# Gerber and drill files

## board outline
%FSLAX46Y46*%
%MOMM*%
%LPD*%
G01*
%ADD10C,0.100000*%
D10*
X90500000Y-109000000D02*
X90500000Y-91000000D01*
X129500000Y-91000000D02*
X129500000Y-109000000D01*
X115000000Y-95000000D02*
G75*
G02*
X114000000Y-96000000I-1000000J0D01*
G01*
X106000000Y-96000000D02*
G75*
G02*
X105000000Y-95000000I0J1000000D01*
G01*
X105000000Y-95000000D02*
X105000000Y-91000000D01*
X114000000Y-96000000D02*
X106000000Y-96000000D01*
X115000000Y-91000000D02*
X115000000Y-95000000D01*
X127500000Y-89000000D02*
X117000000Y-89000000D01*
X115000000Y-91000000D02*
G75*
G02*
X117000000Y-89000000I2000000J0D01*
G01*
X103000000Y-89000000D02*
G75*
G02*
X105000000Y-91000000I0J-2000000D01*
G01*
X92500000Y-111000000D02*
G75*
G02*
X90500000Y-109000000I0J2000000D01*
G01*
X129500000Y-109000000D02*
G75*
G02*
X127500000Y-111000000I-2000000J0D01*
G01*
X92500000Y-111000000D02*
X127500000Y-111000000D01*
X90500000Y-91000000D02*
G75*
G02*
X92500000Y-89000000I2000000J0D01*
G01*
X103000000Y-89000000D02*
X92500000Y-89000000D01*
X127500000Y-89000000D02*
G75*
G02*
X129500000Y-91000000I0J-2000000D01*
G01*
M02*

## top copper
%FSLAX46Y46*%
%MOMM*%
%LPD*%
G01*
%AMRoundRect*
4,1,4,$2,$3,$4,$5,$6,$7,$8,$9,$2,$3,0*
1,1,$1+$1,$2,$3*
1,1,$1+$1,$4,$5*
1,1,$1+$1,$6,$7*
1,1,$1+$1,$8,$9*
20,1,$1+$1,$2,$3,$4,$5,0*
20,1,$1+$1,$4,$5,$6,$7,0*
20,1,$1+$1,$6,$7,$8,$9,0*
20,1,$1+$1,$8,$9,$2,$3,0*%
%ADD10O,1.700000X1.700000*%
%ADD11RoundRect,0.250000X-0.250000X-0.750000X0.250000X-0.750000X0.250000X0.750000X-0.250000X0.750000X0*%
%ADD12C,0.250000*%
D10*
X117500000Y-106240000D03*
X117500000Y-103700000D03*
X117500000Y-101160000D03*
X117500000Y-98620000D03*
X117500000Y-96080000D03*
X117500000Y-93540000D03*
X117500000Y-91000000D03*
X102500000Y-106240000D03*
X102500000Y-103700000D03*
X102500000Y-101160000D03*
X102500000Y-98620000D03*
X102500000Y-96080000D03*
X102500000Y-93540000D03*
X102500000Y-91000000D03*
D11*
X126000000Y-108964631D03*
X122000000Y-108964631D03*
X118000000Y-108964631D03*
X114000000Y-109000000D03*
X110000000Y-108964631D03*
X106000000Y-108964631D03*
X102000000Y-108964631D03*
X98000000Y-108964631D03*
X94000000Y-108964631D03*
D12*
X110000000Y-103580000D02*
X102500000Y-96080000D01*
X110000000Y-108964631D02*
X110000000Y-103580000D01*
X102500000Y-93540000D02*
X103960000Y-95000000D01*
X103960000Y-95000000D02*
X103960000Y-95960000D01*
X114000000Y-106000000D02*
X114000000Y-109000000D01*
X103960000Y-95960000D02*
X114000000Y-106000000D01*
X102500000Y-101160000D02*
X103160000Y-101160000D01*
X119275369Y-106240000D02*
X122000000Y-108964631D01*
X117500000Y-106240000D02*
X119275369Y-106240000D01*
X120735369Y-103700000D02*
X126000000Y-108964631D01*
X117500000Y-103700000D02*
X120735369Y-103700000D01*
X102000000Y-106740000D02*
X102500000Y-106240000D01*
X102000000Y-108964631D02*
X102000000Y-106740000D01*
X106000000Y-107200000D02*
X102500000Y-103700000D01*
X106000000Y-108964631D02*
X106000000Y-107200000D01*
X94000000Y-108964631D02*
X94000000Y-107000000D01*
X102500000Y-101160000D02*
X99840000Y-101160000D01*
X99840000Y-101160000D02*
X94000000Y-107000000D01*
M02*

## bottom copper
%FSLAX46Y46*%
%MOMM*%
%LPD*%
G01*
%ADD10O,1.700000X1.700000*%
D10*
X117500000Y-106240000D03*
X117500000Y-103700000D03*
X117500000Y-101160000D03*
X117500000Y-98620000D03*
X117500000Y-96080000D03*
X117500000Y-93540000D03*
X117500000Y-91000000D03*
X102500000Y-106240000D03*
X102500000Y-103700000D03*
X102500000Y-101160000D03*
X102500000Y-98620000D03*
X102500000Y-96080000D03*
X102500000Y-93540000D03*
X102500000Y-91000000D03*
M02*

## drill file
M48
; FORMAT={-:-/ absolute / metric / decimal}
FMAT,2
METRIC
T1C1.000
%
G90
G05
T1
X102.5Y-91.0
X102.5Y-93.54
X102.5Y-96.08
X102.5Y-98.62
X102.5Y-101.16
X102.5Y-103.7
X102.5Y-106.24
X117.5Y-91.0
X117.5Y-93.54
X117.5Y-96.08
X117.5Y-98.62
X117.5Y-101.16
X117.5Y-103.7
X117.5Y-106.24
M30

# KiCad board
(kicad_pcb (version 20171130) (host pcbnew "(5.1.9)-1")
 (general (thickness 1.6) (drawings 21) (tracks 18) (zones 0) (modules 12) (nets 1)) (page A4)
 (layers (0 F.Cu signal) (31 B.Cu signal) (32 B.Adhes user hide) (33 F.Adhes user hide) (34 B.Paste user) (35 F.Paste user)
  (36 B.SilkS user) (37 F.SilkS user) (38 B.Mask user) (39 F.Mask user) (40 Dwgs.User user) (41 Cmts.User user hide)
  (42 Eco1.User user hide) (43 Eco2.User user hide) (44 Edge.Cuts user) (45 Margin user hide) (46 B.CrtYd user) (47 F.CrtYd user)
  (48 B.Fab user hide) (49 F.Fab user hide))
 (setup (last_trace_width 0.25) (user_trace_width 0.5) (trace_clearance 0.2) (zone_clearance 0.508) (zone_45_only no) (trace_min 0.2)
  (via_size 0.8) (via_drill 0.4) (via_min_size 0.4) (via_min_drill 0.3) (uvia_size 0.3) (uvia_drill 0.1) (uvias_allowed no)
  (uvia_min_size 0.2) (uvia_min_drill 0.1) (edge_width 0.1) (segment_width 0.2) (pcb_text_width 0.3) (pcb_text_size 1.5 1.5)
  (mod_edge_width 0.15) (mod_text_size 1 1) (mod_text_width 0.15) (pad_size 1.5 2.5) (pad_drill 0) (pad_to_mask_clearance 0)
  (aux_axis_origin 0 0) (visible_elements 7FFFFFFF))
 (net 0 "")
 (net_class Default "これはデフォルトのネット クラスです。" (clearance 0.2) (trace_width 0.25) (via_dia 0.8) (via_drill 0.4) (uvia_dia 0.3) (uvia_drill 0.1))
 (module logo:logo (layer F.Cu) (at 96.5 99 90)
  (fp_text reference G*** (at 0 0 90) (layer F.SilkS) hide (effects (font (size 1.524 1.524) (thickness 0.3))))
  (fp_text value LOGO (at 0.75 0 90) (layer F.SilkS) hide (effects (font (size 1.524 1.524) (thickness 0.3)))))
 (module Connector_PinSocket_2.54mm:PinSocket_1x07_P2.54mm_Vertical (layer F.Cu) (at 117.5 91)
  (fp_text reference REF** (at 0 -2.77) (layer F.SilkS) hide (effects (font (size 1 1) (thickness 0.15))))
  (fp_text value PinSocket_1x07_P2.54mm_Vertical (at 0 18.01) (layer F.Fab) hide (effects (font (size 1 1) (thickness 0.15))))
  (pad 7 thru_hole oval (at 0 15.24) (size 1.7 1.7) (drill 1) (layers *.Cu *.Mask))
  (pad 6 thru_hole oval (at 0 12.7) (size 1.7 1.7) (drill 1) (layers *.Cu *.Mask))
  (pad 5 thru_hole oval (at 0 10.16) (size 1.7 1.7) (drill 1) (layers *.Cu *.Mask))
  (pad 4 thru_hole oval (at 0 7.62) (size 1.7 1.7) (drill 1) (layers *.Cu *.Mask))
  (pad 3 thru_hole oval (at 0 5.08) (size 1.7 1.7) (drill 1) (layers *.Cu *.Mask))
  (pad 2 thru_hole oval (at 0 2.54) (size 1.7 1.7) (drill 1) (layers *.Cu *.Mask))
  (pad 1 thru_hole oval (at 0 0) (size 1.7 1.7) (drill 1) (layers *.Cu *.Mask)))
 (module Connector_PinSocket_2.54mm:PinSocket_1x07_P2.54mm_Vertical (layer F.Cu) (at 102.5 91)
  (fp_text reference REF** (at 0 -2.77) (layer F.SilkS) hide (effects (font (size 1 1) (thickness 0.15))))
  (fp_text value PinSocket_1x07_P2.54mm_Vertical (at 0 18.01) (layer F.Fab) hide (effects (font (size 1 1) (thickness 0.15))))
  (pad 8 thru_hole oval (at 0 15.24) (size 1.7 1.7) (drill 1) (layers *.Cu *.Mask))
  (pad 9 thru_hole oval (at 0 12.7) (size 1.7 1.7) (drill 1) (layers *.Cu *.Mask))
  (pad 10 thru_hole oval (at 0 10.16) (size 1.7 1.7) (drill 1) (layers *.Cu *.Mask))
  (pad 11 thru_hole oval (at 0 7.62) (size 1.7 1.7) (drill 1) (layers *.Cu *.Mask))
  (pad 12 thru_hole oval (at 0 5.08) (size 1.7 1.7) (drill 1) (layers *.Cu *.Mask))
  (pad 13 thru_hole oval (at 0 2.54) (size 1.7 1.7) (drill 1) (layers *.Cu *.Mask))
  (pad 14 thru_hole oval (at 0 0) (size 1.7 1.7) (drill 1) (layers *.Cu *.Mask)))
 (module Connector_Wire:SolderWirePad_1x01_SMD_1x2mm (layer F.Cu) (at 126 108.964631)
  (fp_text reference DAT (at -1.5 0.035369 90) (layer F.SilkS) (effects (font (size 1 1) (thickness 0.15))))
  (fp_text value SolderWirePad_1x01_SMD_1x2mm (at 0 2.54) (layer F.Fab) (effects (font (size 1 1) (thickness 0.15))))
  (pad 9 smd roundrect (at 0 0) (size 1 2) (layers F.Cu F.Paste F.Mask) (roundrect_rratio 0.25)))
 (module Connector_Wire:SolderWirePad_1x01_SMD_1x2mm (layer F.Cu) (at 122 108.964631)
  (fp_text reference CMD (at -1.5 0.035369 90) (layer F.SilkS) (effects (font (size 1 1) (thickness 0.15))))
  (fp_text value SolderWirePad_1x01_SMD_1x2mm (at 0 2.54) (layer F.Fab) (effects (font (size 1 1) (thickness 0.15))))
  (pad 8 smd roundrect (at 0 0) (size 1 2) (layers F.Cu F.Paste F.Mask) (roundrect_rratio 0.25)))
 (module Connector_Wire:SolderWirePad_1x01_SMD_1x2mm (layer F.Cu) (at 118 108.964631)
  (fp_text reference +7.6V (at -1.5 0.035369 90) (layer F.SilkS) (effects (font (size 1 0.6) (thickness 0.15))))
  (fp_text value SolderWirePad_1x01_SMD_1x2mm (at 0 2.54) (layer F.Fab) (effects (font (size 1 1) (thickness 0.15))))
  (pad 7 smd roundrect (at 0 0) (size 1 2) (layers F.Cu F.Paste F.Mask) (roundrect_rratio 0.25)))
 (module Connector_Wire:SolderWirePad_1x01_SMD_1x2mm (layer F.Cu) (at 114 109)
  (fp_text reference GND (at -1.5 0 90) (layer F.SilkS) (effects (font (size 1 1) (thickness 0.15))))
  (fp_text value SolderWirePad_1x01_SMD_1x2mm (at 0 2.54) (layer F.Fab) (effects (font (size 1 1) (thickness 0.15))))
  (pad 6 smd roundrect (at 0 0) (size 1 2) (layers F.Cu F.Paste F.Mask) (roundrect_rratio 0.25)))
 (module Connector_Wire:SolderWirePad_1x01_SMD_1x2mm (layer F.Cu) (at 110 108.964631)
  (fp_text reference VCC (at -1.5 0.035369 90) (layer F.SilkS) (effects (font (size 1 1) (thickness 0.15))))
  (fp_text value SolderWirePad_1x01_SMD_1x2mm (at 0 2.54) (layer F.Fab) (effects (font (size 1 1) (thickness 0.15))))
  (pad 5 smd roundrect (at 0 0) (size 1 2) (layers F.Cu F.Paste F.Mask) (roundrect_rratio 0.25)))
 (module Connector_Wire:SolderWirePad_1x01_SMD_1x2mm (layer F.Cu) (at 106 108.964631)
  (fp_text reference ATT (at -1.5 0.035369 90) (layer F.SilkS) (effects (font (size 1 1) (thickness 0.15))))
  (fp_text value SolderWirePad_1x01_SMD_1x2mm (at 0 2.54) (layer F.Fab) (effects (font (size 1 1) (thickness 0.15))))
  (pad 4 smd roundrect (at 0 0) (size 1 2) (layers F.Cu F.Paste F.Mask) (roundrect_rratio 0.25)))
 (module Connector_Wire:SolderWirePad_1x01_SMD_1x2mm (layer F.Cu) (at 102 108.964631)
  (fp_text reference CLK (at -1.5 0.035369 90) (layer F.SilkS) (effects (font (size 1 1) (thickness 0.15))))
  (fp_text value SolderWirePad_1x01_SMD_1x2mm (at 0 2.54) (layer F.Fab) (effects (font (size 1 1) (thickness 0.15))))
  (pad 3 smd roundrect (at 0 0) (size 1 2) (layers F.Cu F.Paste F.Mask) (roundrect_rratio 0.25)))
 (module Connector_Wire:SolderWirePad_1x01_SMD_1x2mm (layer F.Cu) (at 98 108.964631)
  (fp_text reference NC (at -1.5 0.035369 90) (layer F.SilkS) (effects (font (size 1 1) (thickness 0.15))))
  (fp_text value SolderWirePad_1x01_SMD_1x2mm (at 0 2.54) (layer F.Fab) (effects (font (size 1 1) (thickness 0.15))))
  (pad 2 smd roundrect (at 0 0) (size 1 2) (layers F.Cu F.Paste F.Mask) (roundrect_rratio 0.25)))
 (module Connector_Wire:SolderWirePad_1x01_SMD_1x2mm (layer F.Cu) (at 94 108.964631)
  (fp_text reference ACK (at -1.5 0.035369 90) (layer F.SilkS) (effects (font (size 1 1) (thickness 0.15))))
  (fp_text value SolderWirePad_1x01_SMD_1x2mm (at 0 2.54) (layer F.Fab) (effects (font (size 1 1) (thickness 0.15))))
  (pad 1 smd roundrect (at 0 0) (size 1 2) (layers F.Cu F.Paste F.Mask) (roundrect_rratio 0.25)))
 (gr_line (start 90.5 109) (end 90.5 91) (layer Edge.Cuts) (width 0.1))
 (gr_line (start 129.5 91) (end 129.5 109) (layer Edge.Cuts) (width 0.1))
 (gr_arc (start 114 95) (end 114 96) (angle -90) (layer Edge.Cuts) (width 0.1))
 (gr_arc (start 106 95) (end 106 96) (angle 90) (layer Edge.Cuts) (width 0.1))
 (gr_line (start 105 95) (end 105 91) (layer Edge.Cuts) (width 0.1))
 (gr_line (start 114 96) (end 106 96) (layer Edge.Cuts) (width 0.1))
 (gr_line (start 115 91) (end 115 95) (layer Edge.Cuts) (width 0.1))
 (gr_line (start 127.5 89) (end 117 89) (layer Edge.Cuts) (width 0.1))
 (gr_arc (start 117 91) (end 115 91) (angle 90) (layer Edge.Cuts) (width 0.1))
 (gr_arc (start 103 91) (end 105 91) (angle -90) (layer Edge.Cuts) (width 0.1))
 (gr_arc (start 92.5 109) (end 92.5 111) (angle 90) (layer Edge.Cuts) (width 0.1))
 (gr_arc (start 127.5 109) (end 127.5 111) (angle -90) (layer Edge.Cuts) (width 0.1))
 (gr_line (start 92.5 111) (end 127.5 111) (layer Edge.Cuts) (width 0.1))
 (gr_arc (start 92.5 91) (end 92.5 89) (angle -90) (layer Edge.Cuts) (width 0.1))
 (gr_line (start 103 89) (end 92.5 89) (layer Edge.Cuts) (width 0.1))
 (gr_arc (start 127.5 91) (end 127.5 89) (angle 90) (layer Edge.Cuts) (width 0.1))
 (segment (start 110 103.58) (end 102.5 96.08) (width 0.25) (layer F.Cu) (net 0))
 (segment (start 110 108.964631) (end 110 103.58) (width 0.25) (layer F.Cu) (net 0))
 (segment (start 102.5 93.54) (end 103.96 95) (width 0.25) (layer F.Cu) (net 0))
 (segment (start 103.96 95) (end 103.96 95.96) (width 0.25) (layer F.Cu) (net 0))
 (segment (start 114 106) (end 114 109) (width 0.25) (layer F.Cu) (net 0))
 (segment (start 103.96 95.96) (end 114 106) (width 0.25) (layer F.Cu) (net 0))
 (segment (start 102.5 101.16) (end 103.16 101.16) (width 0.25) (layer F.Cu) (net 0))
 (segment (start 119.275369 106.24) (end 122 108.964631) (width 0.25) (layer F.Cu) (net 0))
 (segment (start 117.5 106.24) (end 119.275369 106.24) (width 0.25) (layer F.Cu) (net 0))
 (segment (start 120.735369 103.7) (end 126 108.964631) (width 0.25) (layer F.Cu) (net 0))
 (segment (start 117.5 103.7) (end 120.735369 103.7) (width 0.25) (layer F.Cu) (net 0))
 (segment (start 102 106.74) (end 102.5 106.24) (width 0.25) (layer F.Cu) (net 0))
 (segment (start 102 108.964631) (end 102 106.74) (width 0.25) (layer F.Cu) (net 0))
 (segment (start 106 107.2) (end 102.5 103.7) (width 0.25) (layer F.Cu) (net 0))
 (segment (start 106 108.964631) (end 106 107.2) (width 0.25) (layer F.Cu) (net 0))
 (segment (start 94 108.964631) (end 94 107) (width 0.25) (layer F.Cu) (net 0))
 (segment (start 102.5 101.16) (end 99.84 101.16) (width 0.25) (layer F.Cu) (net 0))
 (segment (start 99.84 101.16) (end 94 107) (width 0.25) (layer F.Cu) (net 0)))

